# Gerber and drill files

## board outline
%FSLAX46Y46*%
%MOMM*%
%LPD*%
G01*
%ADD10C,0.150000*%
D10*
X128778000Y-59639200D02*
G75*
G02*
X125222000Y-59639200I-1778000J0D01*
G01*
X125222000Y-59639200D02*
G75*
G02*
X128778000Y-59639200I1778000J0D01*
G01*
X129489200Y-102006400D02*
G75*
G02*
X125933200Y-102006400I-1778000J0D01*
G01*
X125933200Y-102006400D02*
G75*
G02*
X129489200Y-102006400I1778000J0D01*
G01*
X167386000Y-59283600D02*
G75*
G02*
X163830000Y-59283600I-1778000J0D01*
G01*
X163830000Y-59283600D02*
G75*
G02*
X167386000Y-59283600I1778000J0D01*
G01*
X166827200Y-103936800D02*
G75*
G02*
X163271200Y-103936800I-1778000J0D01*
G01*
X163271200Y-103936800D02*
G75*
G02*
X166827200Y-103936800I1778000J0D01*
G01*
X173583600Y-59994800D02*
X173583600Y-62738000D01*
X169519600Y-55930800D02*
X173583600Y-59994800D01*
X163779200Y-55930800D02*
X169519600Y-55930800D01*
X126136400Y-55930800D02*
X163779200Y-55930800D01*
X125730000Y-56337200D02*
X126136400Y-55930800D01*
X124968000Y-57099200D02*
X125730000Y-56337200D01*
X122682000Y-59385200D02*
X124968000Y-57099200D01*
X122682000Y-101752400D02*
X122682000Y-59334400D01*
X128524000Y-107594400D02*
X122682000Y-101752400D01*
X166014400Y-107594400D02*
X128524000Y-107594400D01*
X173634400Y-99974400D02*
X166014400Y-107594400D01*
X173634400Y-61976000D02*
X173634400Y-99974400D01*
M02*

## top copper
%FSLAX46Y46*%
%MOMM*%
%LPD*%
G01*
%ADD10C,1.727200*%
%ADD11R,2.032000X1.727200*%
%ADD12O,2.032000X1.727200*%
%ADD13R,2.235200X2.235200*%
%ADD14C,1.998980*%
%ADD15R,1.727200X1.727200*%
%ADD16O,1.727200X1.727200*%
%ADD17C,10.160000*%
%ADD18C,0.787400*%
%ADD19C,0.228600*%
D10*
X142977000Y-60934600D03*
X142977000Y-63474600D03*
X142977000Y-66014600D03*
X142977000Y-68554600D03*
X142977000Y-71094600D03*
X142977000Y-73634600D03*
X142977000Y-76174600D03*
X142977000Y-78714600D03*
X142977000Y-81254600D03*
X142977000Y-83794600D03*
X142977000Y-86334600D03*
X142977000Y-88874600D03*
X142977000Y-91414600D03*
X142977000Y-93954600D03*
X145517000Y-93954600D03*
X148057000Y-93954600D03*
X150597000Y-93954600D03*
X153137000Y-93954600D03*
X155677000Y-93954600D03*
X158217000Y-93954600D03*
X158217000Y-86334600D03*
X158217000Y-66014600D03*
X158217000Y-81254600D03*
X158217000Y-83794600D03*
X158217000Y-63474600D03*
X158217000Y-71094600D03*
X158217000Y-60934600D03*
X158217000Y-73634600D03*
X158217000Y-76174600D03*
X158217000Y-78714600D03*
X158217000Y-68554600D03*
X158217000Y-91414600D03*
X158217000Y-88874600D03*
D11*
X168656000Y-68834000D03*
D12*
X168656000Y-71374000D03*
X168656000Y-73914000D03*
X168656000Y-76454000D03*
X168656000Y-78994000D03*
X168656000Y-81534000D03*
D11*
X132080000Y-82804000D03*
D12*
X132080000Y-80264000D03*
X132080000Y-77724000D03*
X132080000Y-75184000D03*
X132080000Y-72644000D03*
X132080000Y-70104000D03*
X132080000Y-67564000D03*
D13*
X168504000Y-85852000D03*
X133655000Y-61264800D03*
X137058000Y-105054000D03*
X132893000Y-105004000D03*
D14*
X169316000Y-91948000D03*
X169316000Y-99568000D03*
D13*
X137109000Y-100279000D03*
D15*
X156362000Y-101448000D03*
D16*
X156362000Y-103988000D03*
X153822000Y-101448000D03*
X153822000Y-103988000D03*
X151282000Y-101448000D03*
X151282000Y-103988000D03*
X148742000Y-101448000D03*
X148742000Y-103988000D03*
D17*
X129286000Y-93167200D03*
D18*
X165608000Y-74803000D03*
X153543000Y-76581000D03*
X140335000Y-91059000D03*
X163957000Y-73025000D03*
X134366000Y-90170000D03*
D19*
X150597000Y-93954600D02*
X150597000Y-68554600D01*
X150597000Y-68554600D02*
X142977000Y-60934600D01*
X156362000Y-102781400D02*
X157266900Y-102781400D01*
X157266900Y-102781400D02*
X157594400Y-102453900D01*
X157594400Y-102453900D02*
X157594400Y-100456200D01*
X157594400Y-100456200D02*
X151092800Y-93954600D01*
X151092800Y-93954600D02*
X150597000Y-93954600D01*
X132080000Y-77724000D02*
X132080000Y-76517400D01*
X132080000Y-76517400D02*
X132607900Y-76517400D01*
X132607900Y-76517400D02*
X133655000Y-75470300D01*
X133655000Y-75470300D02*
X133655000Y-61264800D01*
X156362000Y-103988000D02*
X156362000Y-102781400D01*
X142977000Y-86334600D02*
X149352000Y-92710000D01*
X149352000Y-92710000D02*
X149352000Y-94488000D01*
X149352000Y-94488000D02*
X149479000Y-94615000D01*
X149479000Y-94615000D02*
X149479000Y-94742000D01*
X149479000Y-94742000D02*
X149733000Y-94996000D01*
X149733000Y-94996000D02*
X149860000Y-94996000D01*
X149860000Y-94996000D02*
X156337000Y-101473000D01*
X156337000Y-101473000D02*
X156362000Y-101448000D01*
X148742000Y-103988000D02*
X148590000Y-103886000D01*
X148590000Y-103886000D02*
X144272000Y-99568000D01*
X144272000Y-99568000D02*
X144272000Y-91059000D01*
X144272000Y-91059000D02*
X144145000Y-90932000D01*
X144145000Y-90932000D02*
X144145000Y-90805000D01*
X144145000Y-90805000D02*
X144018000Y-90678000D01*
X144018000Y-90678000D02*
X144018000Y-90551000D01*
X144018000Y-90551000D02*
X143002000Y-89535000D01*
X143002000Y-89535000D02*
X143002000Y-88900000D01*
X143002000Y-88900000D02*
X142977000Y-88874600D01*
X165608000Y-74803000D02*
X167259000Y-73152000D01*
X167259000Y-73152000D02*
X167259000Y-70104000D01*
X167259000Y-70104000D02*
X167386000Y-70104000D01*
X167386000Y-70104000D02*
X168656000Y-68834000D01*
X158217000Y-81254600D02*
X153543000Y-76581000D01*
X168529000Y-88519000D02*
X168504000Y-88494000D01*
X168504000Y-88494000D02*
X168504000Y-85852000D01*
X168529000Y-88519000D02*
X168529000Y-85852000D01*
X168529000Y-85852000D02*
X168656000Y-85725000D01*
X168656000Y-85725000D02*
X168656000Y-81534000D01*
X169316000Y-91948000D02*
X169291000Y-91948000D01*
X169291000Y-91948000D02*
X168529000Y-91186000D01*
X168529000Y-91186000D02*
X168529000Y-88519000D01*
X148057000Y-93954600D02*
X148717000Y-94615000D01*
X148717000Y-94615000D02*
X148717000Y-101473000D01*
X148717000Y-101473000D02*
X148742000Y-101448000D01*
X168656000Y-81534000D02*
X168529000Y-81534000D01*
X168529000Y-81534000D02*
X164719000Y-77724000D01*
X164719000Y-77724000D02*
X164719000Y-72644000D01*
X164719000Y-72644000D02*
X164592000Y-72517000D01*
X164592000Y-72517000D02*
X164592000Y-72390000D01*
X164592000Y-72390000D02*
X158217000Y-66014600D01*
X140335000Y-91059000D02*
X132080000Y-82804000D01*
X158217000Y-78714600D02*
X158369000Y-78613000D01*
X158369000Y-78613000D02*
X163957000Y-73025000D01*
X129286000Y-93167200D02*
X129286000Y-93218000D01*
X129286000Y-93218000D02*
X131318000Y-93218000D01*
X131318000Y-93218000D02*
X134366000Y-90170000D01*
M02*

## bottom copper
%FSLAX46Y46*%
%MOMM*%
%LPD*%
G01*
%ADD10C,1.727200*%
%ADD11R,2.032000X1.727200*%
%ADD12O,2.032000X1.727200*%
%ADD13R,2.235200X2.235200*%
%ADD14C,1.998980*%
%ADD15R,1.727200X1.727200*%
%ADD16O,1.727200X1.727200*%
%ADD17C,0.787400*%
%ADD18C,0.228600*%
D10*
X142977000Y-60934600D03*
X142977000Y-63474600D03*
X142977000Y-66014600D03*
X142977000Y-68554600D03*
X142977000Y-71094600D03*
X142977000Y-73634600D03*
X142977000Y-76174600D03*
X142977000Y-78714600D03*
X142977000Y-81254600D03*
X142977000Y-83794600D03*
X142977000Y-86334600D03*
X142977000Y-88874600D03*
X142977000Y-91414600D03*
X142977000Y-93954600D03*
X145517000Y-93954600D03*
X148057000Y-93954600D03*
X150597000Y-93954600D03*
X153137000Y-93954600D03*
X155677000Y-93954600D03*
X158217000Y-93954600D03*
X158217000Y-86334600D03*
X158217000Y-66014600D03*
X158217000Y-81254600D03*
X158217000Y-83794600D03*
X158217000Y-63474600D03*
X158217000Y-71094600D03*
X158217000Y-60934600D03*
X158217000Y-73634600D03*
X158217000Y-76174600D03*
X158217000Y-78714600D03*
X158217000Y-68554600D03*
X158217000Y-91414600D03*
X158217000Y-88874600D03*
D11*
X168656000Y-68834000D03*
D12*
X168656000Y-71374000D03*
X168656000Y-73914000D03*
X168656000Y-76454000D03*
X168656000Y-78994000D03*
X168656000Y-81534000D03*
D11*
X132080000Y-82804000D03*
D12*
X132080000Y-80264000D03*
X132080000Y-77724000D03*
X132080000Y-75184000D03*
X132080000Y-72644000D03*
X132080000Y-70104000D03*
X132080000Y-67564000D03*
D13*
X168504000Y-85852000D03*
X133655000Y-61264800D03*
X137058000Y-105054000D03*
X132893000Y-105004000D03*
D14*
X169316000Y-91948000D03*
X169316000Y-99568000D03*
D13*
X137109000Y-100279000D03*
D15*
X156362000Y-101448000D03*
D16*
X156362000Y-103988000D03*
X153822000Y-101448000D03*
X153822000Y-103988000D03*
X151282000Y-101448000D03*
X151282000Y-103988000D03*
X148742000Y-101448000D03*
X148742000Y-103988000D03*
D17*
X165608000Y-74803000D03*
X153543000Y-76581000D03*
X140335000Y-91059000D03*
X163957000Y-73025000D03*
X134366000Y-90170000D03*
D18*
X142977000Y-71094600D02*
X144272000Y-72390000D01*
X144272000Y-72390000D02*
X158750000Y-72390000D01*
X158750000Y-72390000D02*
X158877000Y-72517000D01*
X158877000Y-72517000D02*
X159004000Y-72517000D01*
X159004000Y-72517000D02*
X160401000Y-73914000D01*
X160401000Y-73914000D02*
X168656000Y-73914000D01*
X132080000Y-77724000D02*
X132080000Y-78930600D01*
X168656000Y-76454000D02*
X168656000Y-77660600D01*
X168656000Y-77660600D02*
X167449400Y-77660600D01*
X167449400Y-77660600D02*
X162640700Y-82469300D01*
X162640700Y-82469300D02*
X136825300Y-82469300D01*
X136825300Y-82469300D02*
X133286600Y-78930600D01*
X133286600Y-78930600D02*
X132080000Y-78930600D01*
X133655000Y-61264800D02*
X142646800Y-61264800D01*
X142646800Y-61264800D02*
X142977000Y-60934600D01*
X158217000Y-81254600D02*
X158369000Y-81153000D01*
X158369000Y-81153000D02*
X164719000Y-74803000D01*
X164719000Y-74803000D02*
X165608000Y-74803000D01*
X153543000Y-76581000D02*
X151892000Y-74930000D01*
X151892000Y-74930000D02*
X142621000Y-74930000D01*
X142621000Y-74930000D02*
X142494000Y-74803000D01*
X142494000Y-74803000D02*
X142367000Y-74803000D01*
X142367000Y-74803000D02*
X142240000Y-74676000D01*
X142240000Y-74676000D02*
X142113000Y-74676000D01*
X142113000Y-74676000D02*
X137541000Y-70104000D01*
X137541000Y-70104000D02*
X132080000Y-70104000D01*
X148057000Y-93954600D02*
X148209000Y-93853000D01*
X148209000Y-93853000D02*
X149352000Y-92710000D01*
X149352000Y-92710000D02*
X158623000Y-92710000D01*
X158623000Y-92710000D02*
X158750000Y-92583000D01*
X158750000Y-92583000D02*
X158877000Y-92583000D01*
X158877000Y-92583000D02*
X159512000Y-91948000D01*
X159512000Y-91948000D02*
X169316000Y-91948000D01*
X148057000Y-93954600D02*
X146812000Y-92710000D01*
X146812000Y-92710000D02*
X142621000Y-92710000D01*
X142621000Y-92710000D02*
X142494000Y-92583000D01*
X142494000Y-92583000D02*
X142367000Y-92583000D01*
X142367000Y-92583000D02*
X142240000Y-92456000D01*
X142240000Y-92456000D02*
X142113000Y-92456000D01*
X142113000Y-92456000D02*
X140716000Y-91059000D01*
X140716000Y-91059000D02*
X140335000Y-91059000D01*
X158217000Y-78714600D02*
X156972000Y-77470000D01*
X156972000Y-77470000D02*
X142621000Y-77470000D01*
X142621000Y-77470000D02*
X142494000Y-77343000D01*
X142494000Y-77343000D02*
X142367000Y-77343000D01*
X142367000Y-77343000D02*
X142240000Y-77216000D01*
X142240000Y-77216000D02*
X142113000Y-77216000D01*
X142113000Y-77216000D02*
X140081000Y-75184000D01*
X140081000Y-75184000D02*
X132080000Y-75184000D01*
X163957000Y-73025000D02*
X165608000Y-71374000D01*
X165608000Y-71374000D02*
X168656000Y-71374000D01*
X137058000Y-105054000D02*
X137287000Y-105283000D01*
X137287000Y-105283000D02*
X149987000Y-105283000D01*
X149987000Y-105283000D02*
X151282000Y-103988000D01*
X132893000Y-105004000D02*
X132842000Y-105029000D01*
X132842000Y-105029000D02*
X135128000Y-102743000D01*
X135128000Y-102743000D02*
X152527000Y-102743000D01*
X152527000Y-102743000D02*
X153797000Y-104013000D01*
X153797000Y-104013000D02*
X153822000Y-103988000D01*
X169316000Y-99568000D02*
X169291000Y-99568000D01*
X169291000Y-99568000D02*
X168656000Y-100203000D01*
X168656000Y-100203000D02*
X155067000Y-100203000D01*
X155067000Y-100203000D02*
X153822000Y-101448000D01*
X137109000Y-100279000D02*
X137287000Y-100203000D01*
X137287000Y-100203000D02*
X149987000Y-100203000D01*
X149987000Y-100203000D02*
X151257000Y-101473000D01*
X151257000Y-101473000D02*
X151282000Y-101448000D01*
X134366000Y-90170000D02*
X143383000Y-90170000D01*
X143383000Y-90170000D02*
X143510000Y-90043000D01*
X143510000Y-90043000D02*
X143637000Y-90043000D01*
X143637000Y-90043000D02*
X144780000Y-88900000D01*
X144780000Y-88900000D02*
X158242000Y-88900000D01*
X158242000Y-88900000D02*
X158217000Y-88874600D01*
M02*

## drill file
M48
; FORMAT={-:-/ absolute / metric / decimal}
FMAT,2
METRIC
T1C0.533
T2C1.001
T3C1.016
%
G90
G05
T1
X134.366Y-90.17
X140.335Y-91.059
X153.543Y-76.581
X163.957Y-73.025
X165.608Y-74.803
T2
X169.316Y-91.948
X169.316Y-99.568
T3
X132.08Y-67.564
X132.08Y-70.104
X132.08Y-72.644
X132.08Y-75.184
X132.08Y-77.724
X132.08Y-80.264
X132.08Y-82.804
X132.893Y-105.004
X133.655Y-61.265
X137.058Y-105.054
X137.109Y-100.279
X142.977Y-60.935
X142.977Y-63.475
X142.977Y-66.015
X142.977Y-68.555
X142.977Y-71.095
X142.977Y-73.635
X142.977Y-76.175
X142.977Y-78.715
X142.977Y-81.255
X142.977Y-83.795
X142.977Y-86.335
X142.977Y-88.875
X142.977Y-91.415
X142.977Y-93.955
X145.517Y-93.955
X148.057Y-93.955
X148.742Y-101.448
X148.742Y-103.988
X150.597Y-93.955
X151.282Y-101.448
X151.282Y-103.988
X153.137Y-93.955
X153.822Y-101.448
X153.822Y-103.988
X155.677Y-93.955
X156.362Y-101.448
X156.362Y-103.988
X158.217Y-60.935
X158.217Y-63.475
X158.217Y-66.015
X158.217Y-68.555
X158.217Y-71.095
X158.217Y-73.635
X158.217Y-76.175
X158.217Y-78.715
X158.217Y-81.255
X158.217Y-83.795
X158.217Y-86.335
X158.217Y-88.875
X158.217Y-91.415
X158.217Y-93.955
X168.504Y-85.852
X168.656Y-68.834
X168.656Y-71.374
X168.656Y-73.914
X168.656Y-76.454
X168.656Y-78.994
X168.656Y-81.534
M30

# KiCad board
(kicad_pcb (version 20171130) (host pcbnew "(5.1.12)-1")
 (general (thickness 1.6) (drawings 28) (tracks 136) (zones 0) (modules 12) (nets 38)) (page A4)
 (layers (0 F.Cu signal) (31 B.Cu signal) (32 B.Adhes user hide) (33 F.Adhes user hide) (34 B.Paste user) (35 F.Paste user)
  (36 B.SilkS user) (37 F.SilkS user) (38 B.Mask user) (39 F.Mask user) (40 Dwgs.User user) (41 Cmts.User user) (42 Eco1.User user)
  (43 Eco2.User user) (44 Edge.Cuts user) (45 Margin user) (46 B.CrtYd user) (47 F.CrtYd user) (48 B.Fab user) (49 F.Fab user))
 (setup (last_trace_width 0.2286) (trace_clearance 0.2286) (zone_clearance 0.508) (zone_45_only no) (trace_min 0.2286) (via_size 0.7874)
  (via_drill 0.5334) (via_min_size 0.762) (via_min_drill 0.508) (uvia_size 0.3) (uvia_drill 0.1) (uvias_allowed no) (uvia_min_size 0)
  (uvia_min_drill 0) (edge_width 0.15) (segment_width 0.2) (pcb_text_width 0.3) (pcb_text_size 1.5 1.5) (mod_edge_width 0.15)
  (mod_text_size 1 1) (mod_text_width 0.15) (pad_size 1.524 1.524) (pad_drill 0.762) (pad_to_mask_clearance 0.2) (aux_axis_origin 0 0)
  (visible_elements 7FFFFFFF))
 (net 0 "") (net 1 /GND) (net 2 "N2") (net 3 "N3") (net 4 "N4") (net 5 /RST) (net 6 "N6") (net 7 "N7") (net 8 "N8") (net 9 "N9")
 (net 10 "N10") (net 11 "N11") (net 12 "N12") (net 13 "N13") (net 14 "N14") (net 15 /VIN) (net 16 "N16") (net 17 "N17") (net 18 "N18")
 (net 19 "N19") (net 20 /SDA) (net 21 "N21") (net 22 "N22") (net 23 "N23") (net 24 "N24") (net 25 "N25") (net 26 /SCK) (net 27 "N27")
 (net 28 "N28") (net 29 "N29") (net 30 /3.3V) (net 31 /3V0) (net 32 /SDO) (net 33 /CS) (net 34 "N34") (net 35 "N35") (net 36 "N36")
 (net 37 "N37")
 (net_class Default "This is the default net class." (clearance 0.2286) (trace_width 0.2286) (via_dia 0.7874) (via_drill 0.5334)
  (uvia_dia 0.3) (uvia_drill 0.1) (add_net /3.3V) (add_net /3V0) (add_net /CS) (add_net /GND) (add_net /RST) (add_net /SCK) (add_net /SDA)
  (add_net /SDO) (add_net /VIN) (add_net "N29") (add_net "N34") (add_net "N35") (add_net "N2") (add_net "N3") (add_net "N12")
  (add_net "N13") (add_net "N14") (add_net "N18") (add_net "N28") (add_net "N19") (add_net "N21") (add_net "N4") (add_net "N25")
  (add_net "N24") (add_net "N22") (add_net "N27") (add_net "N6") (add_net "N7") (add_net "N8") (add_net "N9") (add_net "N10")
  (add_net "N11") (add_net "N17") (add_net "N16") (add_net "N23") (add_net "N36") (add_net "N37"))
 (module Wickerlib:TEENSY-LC (layer F.Cu) (at 153.137 71.0946)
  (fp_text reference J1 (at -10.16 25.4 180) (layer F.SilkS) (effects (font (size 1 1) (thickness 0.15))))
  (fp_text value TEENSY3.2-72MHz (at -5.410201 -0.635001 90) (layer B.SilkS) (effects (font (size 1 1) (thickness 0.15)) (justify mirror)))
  (pad G1 thru_hole circle (at -10.16 -10.16) (size 1.7272 1.7272) (drill 1.016) (layers *.Cu *.Mask F.SilkS) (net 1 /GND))
  (pad 0 thru_hole circle (at -10.16 -7.62) (size 1.7272 1.7272) (drill 1.016) (layers *.Cu *.Mask F.SilkS) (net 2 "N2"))
  (pad 1 thru_hole circle (at -10.16 -5.08) (size 1.7272 1.7272) (drill 1.016) (layers *.Cu *.Mask F.SilkS) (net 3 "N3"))
  (pad 2 thru_hole circle (at -10.16 -2.54) (size 1.7272 1.7272) (drill 1.016) (layers *.Cu *.Mask F.SilkS) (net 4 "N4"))
  (pad 3 thru_hole circle (at -10.16 0) (size 1.7272 1.7272) (drill 1.016) (layers *.Cu *.Mask F.SilkS) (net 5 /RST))
  (pad 4 thru_hole circle (at -10.16 2.54) (size 1.7272 1.7272) (drill 1.016) (layers *.Cu *.Mask F.SilkS) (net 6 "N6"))
  (pad 5 thru_hole circle (at -10.16 5.08) (size 1.7272 1.7272) (drill 1.016) (layers *.Cu *.Mask F.SilkS) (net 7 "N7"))
  (pad 6 thru_hole circle (at -10.16 7.62) (size 1.7272 1.7272) (drill 1.016) (layers *.Cu *.Mask F.SilkS) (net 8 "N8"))
  (pad 7 thru_hole circle (at -10.16 10.16) (size 1.7272 1.7272) (drill 1.016) (layers *.Cu *.Mask F.SilkS) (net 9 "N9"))
  (pad 8 thru_hole circle (at -10.16 12.7) (size 1.7272 1.7272) (drill 1.016) (layers *.Cu *.Mask F.SilkS) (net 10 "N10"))
  (pad 9 thru_hole circle (at -10.16 15.24) (size 1.7272 1.7272) (drill 1.016) (layers *.Cu *.Mask F.SilkS) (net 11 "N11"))
  (pad 10 thru_hole circle (at -10.16 17.78) (size 1.7272 1.7272) (drill 1.016) (layers *.Cu *.Mask F.SilkS) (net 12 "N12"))
  (pad 11 thru_hole circle (at -10.16 20.32) (size 1.7272 1.7272) (drill 1.016) (layers *.Cu *.Mask F.SilkS) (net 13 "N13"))
  (pad 12 thru_hole circle (at -10.16 22.86) (size 1.7272 1.7272) (drill 1.016) (layers *.Cu *.Mask F.SilkS) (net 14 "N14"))
  (pad 17A thru_hole circle (at -7.62 22.86) (size 1.7272 1.7272) (drill 1.016) (layers *.Cu *.Mask F.SilkS))
  (pad 3V1 thru_hole circle (at -5.08 22.86) (size 1.7272 1.7272) (drill 1.016) (layers *.Cu *.Mask F.SilkS) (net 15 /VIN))
  (pad G2 thru_hole circle (at -2.54 22.86) (size 1.7272 1.7272) (drill 1.016) (layers *.Cu *.Mask F.SilkS) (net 1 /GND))
  (pad PGM thru_hole circle (at 0 22.86) (size 1.7272 1.7272) (drill 1.016) (layers *.Cu *.Mask F.SilkS) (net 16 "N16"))
  (pad DAC thru_hole circle (at 2.54 22.86) (size 1.7272 1.7272) (drill 1.016) (layers *.Cu *.Mask F.SilkS) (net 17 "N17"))
  (pad 13 thru_hole circle (at 5.08 22.86) (size 1.7272 1.7272) (drill 1.016) (layers *.Cu *.Mask F.SilkS) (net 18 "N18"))
  (pad 16 thru_hole circle (at 5.08 15.24) (size 1.7272 1.7272) (drill 1.016) (layers *.Cu *.Mask F.SilkS) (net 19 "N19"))
  (pad 3V2 thru_hole circle (at 5.08 -5.08) (size 1.7272 1.7272) (drill 1.016) (layers *.Cu *.Mask F.SilkS) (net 15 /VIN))
  (pad 18 thru_hole circle (at 5.08 10.16) (size 1.7272 1.7272) (drill 1.016) (layers *.Cu *.Mask F.SilkS) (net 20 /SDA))
  (pad 17 thru_hole circle (at 5.08 12.7) (size 1.7272 1.7272) (drill 1.016) (layers *.Cu *.Mask F.SilkS) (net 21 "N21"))
  (pad G3 thru_hole circle (at 5.08 -7.62) (size 1.7272 1.7272) (drill 1.016) (layers *.Cu *.Mask F.SilkS))
  (pad 22 thru_hole circle (at 5.08 0) (size 1.7272 1.7272) (drill 1.016) (layers *.Cu *.Mask F.SilkS) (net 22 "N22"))
  (pad VIN thru_hole circle (at 5.08 -10.16) (size 1.7272 1.7272) (drill 1.016) (layers *.Cu *.Mask F.SilkS) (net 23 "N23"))
  (pad 21 thru_hole circle (at 5.08 2.54) (size 1.7272 1.7272) (drill 1.016) (layers *.Cu *.Mask F.SilkS) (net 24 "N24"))
  (pad 20 thru_hole circle (at 5.08 5.08) (size 1.7272 1.7272) (drill 1.016) (layers *.Cu *.Mask F.SilkS) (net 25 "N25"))
  (pad 19 thru_hole circle (at 5.08 7.62) (size 1.7272 1.7272) (drill 1.016) (layers *.Cu *.Mask F.SilkS) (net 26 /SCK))
  (pad 23 thru_hole circle (at 5.08 -2.54) (size 1.7272 1.7272) (drill 1.016) (layers *.Cu *.Mask F.SilkS) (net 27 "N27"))
  (pad 14 thru_hole circle (at 5.08 20.32) (size 1.7272 1.7272) (drill 1.016) (layers *.Cu *.Mask F.SilkS) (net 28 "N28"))
  (pad 15 thru_hole circle (at 5.08 17.78) (size 1.7272 1.7272) (drill 1.016) (layers *.Cu *.Mask F.SilkS) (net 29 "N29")))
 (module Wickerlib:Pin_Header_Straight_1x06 (layer F.Cu) (at 168.656 68.834)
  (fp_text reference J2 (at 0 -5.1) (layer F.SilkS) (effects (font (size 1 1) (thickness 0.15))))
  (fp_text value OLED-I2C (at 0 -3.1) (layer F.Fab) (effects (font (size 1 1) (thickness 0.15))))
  (pad 1 thru_hole rect (at 0 0) (size 2.032 1.7272) (drill 1.016) (layers *.Cu *.Mask F.SilkS) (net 20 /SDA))
  (pad 2 thru_hole oval (at 0 2.54) (size 2.032 1.7272) (drill 1.016) (layers *.Cu *.Mask F.SilkS) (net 26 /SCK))
  (pad 3 thru_hole oval (at 0 5.08) (size 2.032 1.7272) (drill 1.016) (layers *.Cu *.Mask F.SilkS) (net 5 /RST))
  (pad 4 thru_hole oval (at 0 7.62) (size 2.032 1.7272) (drill 1.016) (layers *.Cu *.Mask F.SilkS) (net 1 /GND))
  (pad 5 thru_hole oval (at 0 10.16) (size 2.032 1.7272) (drill 1.016) (layers *.Cu *.Mask F.SilkS) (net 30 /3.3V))
  (pad 6 thru_hole oval (at 0 12.7) (size 2.032 1.7272) (drill 1.016) (layers *.Cu *.Mask F.SilkS) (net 15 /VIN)))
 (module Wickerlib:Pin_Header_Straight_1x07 (layer F.Cu) (at 132.08 82.804 180)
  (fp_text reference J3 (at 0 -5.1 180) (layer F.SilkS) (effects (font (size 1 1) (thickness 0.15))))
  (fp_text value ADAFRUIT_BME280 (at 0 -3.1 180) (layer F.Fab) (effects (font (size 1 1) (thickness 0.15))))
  (pad 1 thru_hole rect (at 0 0 180) (size 2.032 1.7272) (drill 1.016) (layers *.Cu *.Mask F.SilkS) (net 15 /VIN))
  (pad 2 thru_hole oval (at 0 2.54 180) (size 2.032 1.7272) (drill 1.016) (layers *.Cu *.Mask F.SilkS) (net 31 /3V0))
  (pad 3 thru_hole oval (at 0 5.08 180) (size 2.032 1.7272) (drill 1.016) (layers *.Cu *.Mask F.SilkS) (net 1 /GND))
  (pad 4 thru_hole oval (at 0 7.62 180) (size 2.032 1.7272) (drill 1.016) (layers *.Cu *.Mask F.SilkS) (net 26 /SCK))
  (pad 5 thru_hole oval (at 0 10.16 180) (size 2.032 1.7272) (drill 1.016) (layers *.Cu *.Mask F.SilkS) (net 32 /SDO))
  (pad 6 thru_hole oval (at 0 12.7 180) (size 2.032 1.7272) (drill 1.016) (layers *.Cu *.Mask F.SilkS) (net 20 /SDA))
  (pad 7 thru_hole oval (at 0 15.24 180) (size 2.032 1.7272) (drill 1.016) (layers *.Cu *.Mask F.SilkS) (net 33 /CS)))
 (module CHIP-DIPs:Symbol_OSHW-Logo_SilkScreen (layer F.Cu) (at 129.286 93.0148 270)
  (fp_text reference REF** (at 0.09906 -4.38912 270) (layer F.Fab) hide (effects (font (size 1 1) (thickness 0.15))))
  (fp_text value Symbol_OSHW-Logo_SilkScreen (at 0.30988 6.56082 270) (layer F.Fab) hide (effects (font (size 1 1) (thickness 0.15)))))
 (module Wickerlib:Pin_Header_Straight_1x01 (layer F.Cu) (at 168.504 85.852 90)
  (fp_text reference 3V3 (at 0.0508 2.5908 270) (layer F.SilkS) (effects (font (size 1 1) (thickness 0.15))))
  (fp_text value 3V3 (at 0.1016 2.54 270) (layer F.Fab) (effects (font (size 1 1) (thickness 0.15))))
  (pad 1 thru_hole rect (at 0 0 90) (size 2.2352 2.2352) (drill 1.016) (layers *.Cu *.Mask F.SilkS) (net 15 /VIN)))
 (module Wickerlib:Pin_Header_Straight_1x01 (layer F.Cu) (at 133.655 61.2648)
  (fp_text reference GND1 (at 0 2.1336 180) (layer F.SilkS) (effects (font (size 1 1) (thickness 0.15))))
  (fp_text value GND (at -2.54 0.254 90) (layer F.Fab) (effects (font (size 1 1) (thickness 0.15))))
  (pad 1 thru_hole rect (at 0 0) (size 2.2352 2.2352) (drill 1.016) (layers *.Cu *.Mask F.SilkS) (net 1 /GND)))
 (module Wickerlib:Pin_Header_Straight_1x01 (layer F.Cu) (at 137.058 105.054 270)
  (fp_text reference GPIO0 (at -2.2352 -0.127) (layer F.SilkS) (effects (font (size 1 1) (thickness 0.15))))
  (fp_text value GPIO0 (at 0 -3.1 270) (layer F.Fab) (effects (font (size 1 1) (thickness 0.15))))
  (pad 1 thru_hole rect (at 0 0 270) (size 2.2352 2.2352) (drill 1.016) (layers *.Cu *.Mask F.SilkS) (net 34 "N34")))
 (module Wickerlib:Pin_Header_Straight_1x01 (layer F.Cu) (at 132.893 105.004 270)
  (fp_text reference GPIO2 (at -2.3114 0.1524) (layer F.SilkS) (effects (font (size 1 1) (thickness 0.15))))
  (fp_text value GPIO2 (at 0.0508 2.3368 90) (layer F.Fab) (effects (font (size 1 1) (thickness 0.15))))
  (pad 1 thru_hole rect (at 0 0 270) (size 2.2352 2.2352) (drill 1.016) (layers *.Cu *.Mask F.SilkS) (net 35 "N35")))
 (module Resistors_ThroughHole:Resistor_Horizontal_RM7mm (layer F.Cu) (at 169.316 91.948 270)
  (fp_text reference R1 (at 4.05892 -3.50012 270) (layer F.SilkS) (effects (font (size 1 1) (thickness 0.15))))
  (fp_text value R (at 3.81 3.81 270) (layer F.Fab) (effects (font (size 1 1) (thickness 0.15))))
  (pad 1 thru_hole circle (at 0 0 270) (size 1.99898 1.99898) (drill 1.00076) (layers *.Cu *.SilkS *.Mask) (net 15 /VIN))
  (pad 2 thru_hole circle (at 7.62 0 270) (size 1.99898 1.99898) (drill 1.00076) (layers *.Cu *.SilkS *.Mask) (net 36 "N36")))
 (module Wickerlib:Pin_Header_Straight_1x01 (layer F.Cu) (at 137.109 100.279 270)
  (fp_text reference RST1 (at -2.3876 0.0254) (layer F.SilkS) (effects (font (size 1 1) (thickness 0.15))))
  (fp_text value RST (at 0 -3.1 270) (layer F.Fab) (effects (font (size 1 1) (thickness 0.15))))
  (pad 1 thru_hole rect (at 0 0 270) (size 2.2352 2.2352) (drill 1.016) (layers *.Cu *.Mask F.SilkS) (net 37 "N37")))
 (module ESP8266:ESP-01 (layer F.Cu) (at 156.362 101.448 270)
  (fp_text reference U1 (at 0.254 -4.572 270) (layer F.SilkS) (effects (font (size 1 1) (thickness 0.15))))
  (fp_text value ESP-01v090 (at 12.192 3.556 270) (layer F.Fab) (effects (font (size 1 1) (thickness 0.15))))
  (pad 1 thru_hole rect (at 0 0 270) (size 1.7272 1.7272) (drill 1.016) (layers *.Cu *.Mask F.SilkS) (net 11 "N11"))
  (pad 2 thru_hole oval (at 2.54 0 270) (size 1.7272 1.7272) (drill 1.016) (layers *.Cu *.Mask F.SilkS) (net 1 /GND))
  (pad 3 thru_hole oval (at 0 2.54 270) (size 1.7272 1.7272) (drill 1.016) (layers *.Cu *.Mask F.SilkS) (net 36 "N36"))
  (pad 4 thru_hole oval (at 2.54 2.54 270) (size 1.7272 1.7272) (drill 1.016) (layers *.Cu *.Mask F.SilkS) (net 35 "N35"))
  (pad 5 thru_hole oval (at 0 5.08 270) (size 1.7272 1.7272) (drill 1.016) (layers *.Cu *.Mask F.SilkS) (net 37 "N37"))
  (pad 6 thru_hole oval (at 2.54 5.08 270) (size 1.7272 1.7272) (drill 1.016) (layers *.Cu *.Mask F.SilkS) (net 34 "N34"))
  (pad 7 thru_hole oval (at 0 7.62 270) (size 1.7272 1.7272) (drill 1.016) (layers *.Cu *.Mask F.SilkS) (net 15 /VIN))
  (pad 8 thru_hole oval (at 2.54 7.62 270) (size 1.7272 1.7272) (drill 1.016) (layers *.Cu *.Mask F.SilkS) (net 12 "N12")))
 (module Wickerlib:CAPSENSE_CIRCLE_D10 (layer F.Cu) (at 129.286 93.1672)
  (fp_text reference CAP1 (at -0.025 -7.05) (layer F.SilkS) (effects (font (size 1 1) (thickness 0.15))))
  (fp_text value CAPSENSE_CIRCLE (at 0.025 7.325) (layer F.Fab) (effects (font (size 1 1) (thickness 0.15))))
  (pad 1 smd circle (at 0 0) (size 10.16 10.16) (layers F.Cu) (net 29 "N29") (clearance 0.508)))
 (gr_circle (center 127 59.6392) (end 128.4224 60.706) (layer Edge.Cuts) (width 0.15))
 (gr_circle (center 127.7112 102.0064) (end 129.1336 103.0732) (layer Edge.Cuts) (width 0.15))
 (gr_circle (center 165.608 59.2836) (end 167.0304 60.3504) (layer Edge.Cuts) (width 0.15))
 (gr_circle (center 165.0492 103.9368) (end 166.4716 105.0036) (layer Edge.Cuts) (width 0.15))
 (gr_line (start 173.5836 59.9948) (end 173.5836 62.738) (angle 90) (layer Edge.Cuts) (width 0.15))
 (gr_line (start 169.5196 55.9308) (end 173.5836 59.9948) (angle 90) (layer Edge.Cuts) (width 0.15))
 (gr_line (start 163.7792 55.9308) (end 169.5196 55.9308) (angle 90) (layer Edge.Cuts) (width 0.15))
 (gr_line (start 126.1364 55.9308) (end 163.7792 55.9308) (angle 90) (layer Edge.Cuts) (width 0.15))
 (gr_line (start 125.73 56.3372) (end 126.1364 55.9308) (angle 90) (layer Edge.Cuts) (width 0.15))
 (gr_line (start 124.968 57.0992) (end 125.73 56.3372) (angle 90) (layer Edge.Cuts) (width 0.15))
 (gr_line (start 122.682 59.3852) (end 124.968 57.0992) (angle 90) (layer Edge.Cuts) (width 0.15))
 (gr_line (start 122.682 101.7524) (end 122.682 59.3344) (angle 90) (layer Edge.Cuts) (width 0.15))
 (gr_line (start 128.524 107.5944) (end 122.682 101.7524) (angle 90) (layer Edge.Cuts) (width 0.15))
 (gr_line (start 166.0144 107.5944) (end 128.524 107.5944) (angle 90) (layer Edge.Cuts) (width 0.15))
 (gr_line (start 173.6344 99.9744) (end 166.0144 107.5944) (angle 90) (layer Edge.Cuts) (width 0.15))
 (gr_line (start 173.6344 61.976) (end 173.6344 99.9744) (angle 90) (layer Edge.Cuts) (width 0.15))
 (segment (start 142.977 71.0946) (end 144.272 72.39) (width 0.2286) (layer B.Cu) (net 5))
 (segment (start 144.272 72.39) (end 158.75 72.39) (width 0.2286) (layer B.Cu) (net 5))
 (segment (start 158.75 72.39) (end 158.877 72.517) (width 0.2286) (layer B.Cu) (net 5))
 (segment (start 158.877 72.517) (end 159.004 72.517) (width 0.2286) (layer B.Cu) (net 5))
 (segment (start 159.004 72.517) (end 160.401 73.914) (width 0.2286) (layer B.Cu) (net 5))
 (segment (start 160.401 73.914) (end 168.656 73.914) (width 0.2286) (layer B.Cu) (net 5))
 (segment (start 150.597 93.9546) (end 150.597 68.5546) (width 0.2286) (layer F.Cu) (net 1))
 (segment (start 150.597 68.5546) (end 142.977 60.9346) (width 0.2286) (layer F.Cu) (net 1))
 (segment (start 156.362 102.7814) (end 157.2669 102.7814) (width 0.2286) (layer F.Cu) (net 1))
 (segment (start 157.2669 102.7814) (end 157.5944 102.4539) (width 0.2286) (layer F.Cu) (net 1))
 (segment (start 157.5944 102.4539) (end 157.5944 100.4562) (width 0.2286) (layer F.Cu) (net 1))
 (segment (start 157.5944 100.4562) (end 151.0928 93.9546) (width 0.2286) (layer F.Cu) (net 1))
 (segment (start 151.0928 93.9546) (end 150.597 93.9546) (width 0.2286) (layer F.Cu) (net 1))
 (segment (start 132.08 77.724) (end 132.08 78.9306) (width 0.2286) (layer B.Cu) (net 1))
 (segment (start 168.656 76.454) (end 168.656 77.6606) (width 0.2286) (layer B.Cu) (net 1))
 (segment (start 168.656 77.6606) (end 167.4494 77.6606) (width 0.2286) (layer B.Cu) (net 1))
 (segment (start 167.4494 77.6606) (end 162.6407 82.4693) (width 0.2286) (layer B.Cu) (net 1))
 (segment (start 162.6407 82.4693) (end 136.8253 82.4693) (width 0.2286) (layer B.Cu) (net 1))
 (segment (start 136.8253 82.4693) (end 133.2866 78.9306) (width 0.2286) (layer B.Cu) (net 1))
 (segment (start 133.2866 78.9306) (end 132.08 78.9306) (width 0.2286) (layer B.Cu) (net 1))
 (segment (start 132.08 77.724) (end 132.08 76.5174) (width 0.2286) (layer F.Cu) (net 1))
 (segment (start 132.08 76.5174) (end 132.6079 76.5174) (width 0.2286) (layer F.Cu) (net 1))
 (segment (start 132.6079 76.5174) (end 133.655 75.4703) (width 0.2286) (layer F.Cu) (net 1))
 (segment (start 133.655 75.4703) (end 133.655 61.2648) (width 0.2286) (layer F.Cu) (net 1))
 (segment (start 133.655 61.2648) (end 142.6468 61.2648) (width 0.2286) (layer B.Cu) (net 1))
 (segment (start 142.6468 61.2648) (end 142.977 60.9346) (width 0.2286) (layer B.Cu) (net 1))
 (segment (start 156.362 103.988) (end 156.362 102.7814) (width 0.2286) (layer F.Cu) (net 1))
 (segment (start 142.977 86.3346) (end 149.352 92.71) (width 0.2286) (layer F.Cu) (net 11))
 (segment (start 149.352 92.71) (end 149.352 94.488) (width 0.2286) (layer F.Cu) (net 11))
 (segment (start 149.352 94.488) (end 149.479 94.615) (width 0.2286) (layer F.Cu) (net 11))
 (segment (start 149.479 94.615) (end 149.479 94.742) (width 0.2286) (layer F.Cu) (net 11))
 (segment (start 149.479 94.742) (end 149.733 94.996) (width 0.2286) (layer F.Cu) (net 11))
 (segment (start 149.733 94.996) (end 149.86 94.996) (width 0.2286) (layer F.Cu) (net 11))
 (segment (start 149.86 94.996) (end 156.337 101.473) (width 0.2286) (layer F.Cu) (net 11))
 (segment (start 156.337 101.473) (end 156.362 101.448) (width 0.2286) (layer F.Cu) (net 11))
 (segment (start 148.742 103.988) (end 148.59 103.886) (width 0.2286) (layer F.Cu) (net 12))
 (segment (start 148.59 103.886) (end 144.272 99.568) (width 0.2286) (layer F.Cu) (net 12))
 (segment (start 144.272 99.568) (end 144.272 91.059) (width 0.2286) (layer F.Cu) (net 12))
 (segment (start 144.272 91.059) (end 144.145 90.932) (width 0.2286) (layer F.Cu) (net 12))
 (segment (start 144.145 90.932) (end 144.145 90.805) (width 0.2286) (layer F.Cu) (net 12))
 (segment (start 144.145 90.805) (end 144.018 90.678) (width 0.2286) (layer F.Cu) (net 12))
 (segment (start 144.018 90.678) (end 144.018 90.551) (width 0.2286) (layer F.Cu) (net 12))
 (segment (start 144.018 90.551) (end 143.002 89.535) (width 0.2286) (layer F.Cu) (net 12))
 (segment (start 143.002 89.535) (end 143.002 88.9) (width 0.2286) (layer F.Cu) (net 12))
 (segment (start 143.002 88.9) (end 142.977 88.8746) (width 0.2286) (layer F.Cu) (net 12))
 (segment (start 165.608 74.803) (end 167.259 73.152) (width 0.2286) (layer F.Cu) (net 20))
 (segment (start 167.259 73.152) (end 167.259 70.104) (width 0.2286) (layer F.Cu) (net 20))
 (segment (start 167.259 70.104) (end 167.386 70.104) (width 0.2286) (layer F.Cu) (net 20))
 (segment (start 167.386 70.104) (end 168.656 68.834) (width 0.2286) (layer F.Cu) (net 20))
 (segment (start 158.217 81.2546) (end 158.369 81.153) (width 0.2286) (layer B.Cu) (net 20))
 (segment (start 158.369 81.153) (end 164.719 74.803) (width 0.2286) (layer B.Cu) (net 20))
 (segment (start 164.719 74.803) (end 165.608 74.803) (width 0.2286) (layer B.Cu) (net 20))
 (segment (start 153.543 76.581) (end 151.892 74.93) (width 0.2286) (layer B.Cu) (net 20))
 (segment (start 151.892 74.93) (end 142.621 74.93) (width 0.2286) (layer B.Cu) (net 20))
 (segment (start 142.621 74.93) (end 142.494 74.803) (width 0.2286) (layer B.Cu) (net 20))
 (segment (start 142.494 74.803) (end 142.367 74.803) (width 0.2286) (layer B.Cu) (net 20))
 (segment (start 142.367 74.803) (end 142.24 74.676) (width 0.2286) (layer B.Cu) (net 20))
 (segment (start 142.24 74.676) (end 142.113 74.676) (width 0.2286) (layer B.Cu) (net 20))
 (segment (start 142.113 74.676) (end 137.541 70.104) (width 0.2286) (layer B.Cu) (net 20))
 (segment (start 137.541 70.104) (end 132.08 70.104) (width 0.2286) (layer B.Cu) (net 20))
 (segment (start 158.217 81.2546) (end 153.543 76.581) (width 0.2286) (layer F.Cu) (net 20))
 (via (at 165.608 74.803) (size 0.7874) (layers F.Cu B.Cu) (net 20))
 (via (at 153.543 76.581) (size 0.7874) (layers F.Cu B.Cu) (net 20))
 (segment (start 168.529 88.519) (end 168.504 88.494) (width 0.2286) (layer F.Cu) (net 15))
 (segment (start 168.504 88.494) (end 168.504 85.852) (width 0.2286) (layer F.Cu) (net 15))
 (segment (start 168.529 88.519) (end 168.529 85.852) (width 0.2286) (layer F.Cu) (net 15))
 (segment (start 168.529 85.852) (end 168.656 85.725) (width 0.2286) (layer F.Cu) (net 15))
 (segment (start 168.656 85.725) (end 168.656 81.534) (width 0.2286) (layer F.Cu) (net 15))
 (segment (start 169.316 91.948) (end 169.291 91.948) (width 0.2286) (layer F.Cu) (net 15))
 (segment (start 169.291 91.948) (end 168.529 91.186) (width 0.2286) (layer F.Cu) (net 15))
 (segment (start 168.529 91.186) (end 168.529 88.519) (width 0.2286) (layer F.Cu) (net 15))
 (segment (start 148.057 93.9546) (end 148.717 94.615) (width 0.2286) (layer F.Cu) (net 15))
 (segment (start 148.717 94.615) (end 148.717 101.473) (width 0.2286) (layer F.Cu) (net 15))
 (segment (start 148.717 101.473) (end 148.742 101.448) (width 0.2286) (layer F.Cu) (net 15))
 (segment (start 148.057 93.9546) (end 148.209 93.853) (width 0.2286) (layer B.Cu) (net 15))
 (segment (start 148.209 93.853) (end 149.352 92.71) (width 0.2286) (layer B.Cu) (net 15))
 (segment (start 149.352 92.71) (end 158.623 92.71) (width 0.2286) (layer B.Cu) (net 15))
 (segment (start 158.623 92.71) (end 158.75 92.583) (width 0.2286) (layer B.Cu) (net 15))
 (segment (start 158.75 92.583) (end 158.877 92.583) (width 0.2286) (layer B.Cu) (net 15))
 (segment (start 158.877 92.583) (end 159.512 91.948) (width 0.2286) (layer B.Cu) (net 15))
 (segment (start 159.512 91.948) (end 169.316 91.948) (width 0.2286) (layer B.Cu) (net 15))
 (segment (start 168.656 81.534) (end 168.529 81.534) (width 0.2286) (layer F.Cu) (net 15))
 (segment (start 168.529 81.534) (end 164.719 77.724) (width 0.2286) (layer F.Cu) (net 15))
 (segment (start 164.719 77.724) (end 164.719 72.644) (width 0.2286) (layer F.Cu) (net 15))
 (segment (start 164.719 72.644) (end 164.592 72.517) (width 0.2286) (layer F.Cu) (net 15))
 (segment (start 164.592 72.517) (end 164.592 72.39) (width 0.2286) (layer F.Cu) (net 15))
 (segment (start 164.592 72.39) (end 158.217 66.0146) (width 0.2286) (layer F.Cu) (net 15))
 (segment (start 140.335 91.059) (end 132.08 82.804) (width 0.2286) (layer F.Cu) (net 15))
 (segment (start 148.057 93.9546) (end 146.812 92.71) (width 0.2286) (layer B.Cu) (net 15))
 (segment (start 146.812 92.71) (end 142.621 92.71) (width 0.2286) (layer B.Cu) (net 15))
 (segment (start 142.621 92.71) (end 142.494 92.583) (width 0.2286) (layer B.Cu) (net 15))
 (segment (start 142.494 92.583) (end 142.367 92.583) (width 0.2286) (layer B.Cu) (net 15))
 (segment (start 142.367 92.583) (end 142.24 92.456) (width 0.2286) (layer B.Cu) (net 15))
 (segment (start 142.24 92.456) (end 142.113 92.456) (width 0.2286) (layer B.Cu) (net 15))
 (segment (start 142.113 92.456) (end 140.716 91.059) (width 0.2286) (layer B.Cu) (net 15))
 (segment (start 140.716 91.059) (end 140.335 91.059) (width 0.2286) (layer B.Cu) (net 15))
 (via (at 140.335 91.059) (size 0.7874) (layers F.Cu B.Cu) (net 15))
 (segment (start 158.217 78.7146) (end 156.972 77.47) (width 0.2286) (layer B.Cu) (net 26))
 (segment (start 156.972 77.47) (end 142.621 77.47) (width 0.2286) (layer B.Cu) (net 26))
 (segment (start 142.621 77.47) (end 142.494 77.343) (width 0.2286) (layer B.Cu) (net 26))
 (segment (start 142.494 77.343) (end 142.367 77.343) (width 0.2286) (layer B.Cu) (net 26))
 (segment (start 142.367 77.343) (end 142.24 77.216) (width 0.2286) (layer B.Cu) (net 26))
 (segment (start 142.24 77.216) (end 142.113 77.216) (width 0.2286) (layer B.Cu) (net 26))
 (segment (start 142.113 77.216) (end 140.081 75.184) (width 0.2286) (layer B.Cu) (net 26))
 (segment (start 140.081 75.184) (end 132.08 75.184) (width 0.2286) (layer B.Cu) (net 26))
 (segment (start 163.957 73.025) (end 165.608 71.374) (width 0.2286) (layer B.Cu) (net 26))
 (segment (start 165.608 71.374) (end 168.656 71.374) (width 0.2286) (layer B.Cu) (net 26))
 (segment (start 158.217 78.7146) (end 158.369 78.613) (width 0.2286) (layer F.Cu) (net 26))
 (segment (start 158.369 78.613) (end 163.957 73.025) (width 0.2286) (layer F.Cu) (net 26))
 (via (at 163.957 73.025) (size 0.7874) (layers F.Cu B.Cu) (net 26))
 (segment (start 137.058 105.054) (end 137.287 105.283) (width 0.2286) (layer B.Cu) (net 34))
 (segment (start 137.287 105.283) (end 149.987 105.283) (width 0.2286) (layer B.Cu) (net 34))
 (segment (start 149.987 105.283) (end 151.282 103.988) (width 0.2286) (layer B.Cu) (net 34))
 (segment (start 132.893 105.004) (end 132.842 105.029) (width 0.2286) (layer B.Cu) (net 35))
 (segment (start 132.842 105.029) (end 135.128 102.743) (width 0.2286) (layer B.Cu) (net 35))
 (segment (start 135.128 102.743) (end 152.527 102.743) (width 0.2286) (layer B.Cu) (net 35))
 (segment (start 152.527 102.743) (end 153.797 104.013) (width 0.2286) (layer B.Cu) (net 35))
 (segment (start 153.797 104.013) (end 153.822 103.988) (width 0.2286) (layer B.Cu) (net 35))
 (segment (start 169.316 99.568) (end 169.291 99.568) (width 0.2286) (layer B.Cu) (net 36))
 (segment (start 169.291 99.568) (end 168.656 100.203) (width 0.2286) (layer B.Cu) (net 36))
 (segment (start 168.656 100.203) (end 155.067 100.203) (width 0.2286) (layer B.Cu) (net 36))
 (segment (start 155.067 100.203) (end 153.822 101.448) (width 0.2286) (layer B.Cu) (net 36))
 (segment (start 137.109 100.279) (end 137.287 100.203) (width 0.2286) (layer B.Cu) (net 37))
 (segment (start 137.287 100.203) (end 149.987 100.203) (width 0.2286) (layer B.Cu) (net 37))
 (segment (start 149.987 100.203) (end 151.257 101.473) (width 0.2286) (layer B.Cu) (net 37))
 (segment (start 151.257 101.473) (end 151.282 101.448) (width 0.2286) (layer B.Cu) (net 37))
 (segment (start 134.366 90.17) (end 143.383 90.17) (width 0.2286) (layer B.Cu) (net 29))
 (segment (start 143.383 90.17) (end 143.51 90.043) (width 0.2286) (layer B.Cu) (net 29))
 (segment (start 143.51 90.043) (end 143.637 90.043) (width 0.2286) (layer B.Cu) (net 29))
 (segment (start 143.637 90.043) (end 144.78 88.9) (width 0.2286) (layer B.Cu) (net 29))
 (segment (start 144.78 88.9) (end 158.242 88.9) (width 0.2286) (layer B.Cu) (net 29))
 (segment (start 158.242 88.9) (end 158.217 88.8746) (width 0.2286) (layer B.Cu) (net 29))
 (segment (start 129.286 93.1672) (end 129.286 93.218) (width 0.2286) (layer F.Cu) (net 29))
 (segment (start 129.286 93.218) (end 131.318 93.218) (width 0.2286) (layer F.Cu) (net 29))
 (segment (start 131.318 93.218) (end 134.366 90.17) (width 0.2286) (layer F.Cu) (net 29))
 (via (at 134.366 90.17) (size 0.7874) (layers F.Cu B.Cu) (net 29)))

